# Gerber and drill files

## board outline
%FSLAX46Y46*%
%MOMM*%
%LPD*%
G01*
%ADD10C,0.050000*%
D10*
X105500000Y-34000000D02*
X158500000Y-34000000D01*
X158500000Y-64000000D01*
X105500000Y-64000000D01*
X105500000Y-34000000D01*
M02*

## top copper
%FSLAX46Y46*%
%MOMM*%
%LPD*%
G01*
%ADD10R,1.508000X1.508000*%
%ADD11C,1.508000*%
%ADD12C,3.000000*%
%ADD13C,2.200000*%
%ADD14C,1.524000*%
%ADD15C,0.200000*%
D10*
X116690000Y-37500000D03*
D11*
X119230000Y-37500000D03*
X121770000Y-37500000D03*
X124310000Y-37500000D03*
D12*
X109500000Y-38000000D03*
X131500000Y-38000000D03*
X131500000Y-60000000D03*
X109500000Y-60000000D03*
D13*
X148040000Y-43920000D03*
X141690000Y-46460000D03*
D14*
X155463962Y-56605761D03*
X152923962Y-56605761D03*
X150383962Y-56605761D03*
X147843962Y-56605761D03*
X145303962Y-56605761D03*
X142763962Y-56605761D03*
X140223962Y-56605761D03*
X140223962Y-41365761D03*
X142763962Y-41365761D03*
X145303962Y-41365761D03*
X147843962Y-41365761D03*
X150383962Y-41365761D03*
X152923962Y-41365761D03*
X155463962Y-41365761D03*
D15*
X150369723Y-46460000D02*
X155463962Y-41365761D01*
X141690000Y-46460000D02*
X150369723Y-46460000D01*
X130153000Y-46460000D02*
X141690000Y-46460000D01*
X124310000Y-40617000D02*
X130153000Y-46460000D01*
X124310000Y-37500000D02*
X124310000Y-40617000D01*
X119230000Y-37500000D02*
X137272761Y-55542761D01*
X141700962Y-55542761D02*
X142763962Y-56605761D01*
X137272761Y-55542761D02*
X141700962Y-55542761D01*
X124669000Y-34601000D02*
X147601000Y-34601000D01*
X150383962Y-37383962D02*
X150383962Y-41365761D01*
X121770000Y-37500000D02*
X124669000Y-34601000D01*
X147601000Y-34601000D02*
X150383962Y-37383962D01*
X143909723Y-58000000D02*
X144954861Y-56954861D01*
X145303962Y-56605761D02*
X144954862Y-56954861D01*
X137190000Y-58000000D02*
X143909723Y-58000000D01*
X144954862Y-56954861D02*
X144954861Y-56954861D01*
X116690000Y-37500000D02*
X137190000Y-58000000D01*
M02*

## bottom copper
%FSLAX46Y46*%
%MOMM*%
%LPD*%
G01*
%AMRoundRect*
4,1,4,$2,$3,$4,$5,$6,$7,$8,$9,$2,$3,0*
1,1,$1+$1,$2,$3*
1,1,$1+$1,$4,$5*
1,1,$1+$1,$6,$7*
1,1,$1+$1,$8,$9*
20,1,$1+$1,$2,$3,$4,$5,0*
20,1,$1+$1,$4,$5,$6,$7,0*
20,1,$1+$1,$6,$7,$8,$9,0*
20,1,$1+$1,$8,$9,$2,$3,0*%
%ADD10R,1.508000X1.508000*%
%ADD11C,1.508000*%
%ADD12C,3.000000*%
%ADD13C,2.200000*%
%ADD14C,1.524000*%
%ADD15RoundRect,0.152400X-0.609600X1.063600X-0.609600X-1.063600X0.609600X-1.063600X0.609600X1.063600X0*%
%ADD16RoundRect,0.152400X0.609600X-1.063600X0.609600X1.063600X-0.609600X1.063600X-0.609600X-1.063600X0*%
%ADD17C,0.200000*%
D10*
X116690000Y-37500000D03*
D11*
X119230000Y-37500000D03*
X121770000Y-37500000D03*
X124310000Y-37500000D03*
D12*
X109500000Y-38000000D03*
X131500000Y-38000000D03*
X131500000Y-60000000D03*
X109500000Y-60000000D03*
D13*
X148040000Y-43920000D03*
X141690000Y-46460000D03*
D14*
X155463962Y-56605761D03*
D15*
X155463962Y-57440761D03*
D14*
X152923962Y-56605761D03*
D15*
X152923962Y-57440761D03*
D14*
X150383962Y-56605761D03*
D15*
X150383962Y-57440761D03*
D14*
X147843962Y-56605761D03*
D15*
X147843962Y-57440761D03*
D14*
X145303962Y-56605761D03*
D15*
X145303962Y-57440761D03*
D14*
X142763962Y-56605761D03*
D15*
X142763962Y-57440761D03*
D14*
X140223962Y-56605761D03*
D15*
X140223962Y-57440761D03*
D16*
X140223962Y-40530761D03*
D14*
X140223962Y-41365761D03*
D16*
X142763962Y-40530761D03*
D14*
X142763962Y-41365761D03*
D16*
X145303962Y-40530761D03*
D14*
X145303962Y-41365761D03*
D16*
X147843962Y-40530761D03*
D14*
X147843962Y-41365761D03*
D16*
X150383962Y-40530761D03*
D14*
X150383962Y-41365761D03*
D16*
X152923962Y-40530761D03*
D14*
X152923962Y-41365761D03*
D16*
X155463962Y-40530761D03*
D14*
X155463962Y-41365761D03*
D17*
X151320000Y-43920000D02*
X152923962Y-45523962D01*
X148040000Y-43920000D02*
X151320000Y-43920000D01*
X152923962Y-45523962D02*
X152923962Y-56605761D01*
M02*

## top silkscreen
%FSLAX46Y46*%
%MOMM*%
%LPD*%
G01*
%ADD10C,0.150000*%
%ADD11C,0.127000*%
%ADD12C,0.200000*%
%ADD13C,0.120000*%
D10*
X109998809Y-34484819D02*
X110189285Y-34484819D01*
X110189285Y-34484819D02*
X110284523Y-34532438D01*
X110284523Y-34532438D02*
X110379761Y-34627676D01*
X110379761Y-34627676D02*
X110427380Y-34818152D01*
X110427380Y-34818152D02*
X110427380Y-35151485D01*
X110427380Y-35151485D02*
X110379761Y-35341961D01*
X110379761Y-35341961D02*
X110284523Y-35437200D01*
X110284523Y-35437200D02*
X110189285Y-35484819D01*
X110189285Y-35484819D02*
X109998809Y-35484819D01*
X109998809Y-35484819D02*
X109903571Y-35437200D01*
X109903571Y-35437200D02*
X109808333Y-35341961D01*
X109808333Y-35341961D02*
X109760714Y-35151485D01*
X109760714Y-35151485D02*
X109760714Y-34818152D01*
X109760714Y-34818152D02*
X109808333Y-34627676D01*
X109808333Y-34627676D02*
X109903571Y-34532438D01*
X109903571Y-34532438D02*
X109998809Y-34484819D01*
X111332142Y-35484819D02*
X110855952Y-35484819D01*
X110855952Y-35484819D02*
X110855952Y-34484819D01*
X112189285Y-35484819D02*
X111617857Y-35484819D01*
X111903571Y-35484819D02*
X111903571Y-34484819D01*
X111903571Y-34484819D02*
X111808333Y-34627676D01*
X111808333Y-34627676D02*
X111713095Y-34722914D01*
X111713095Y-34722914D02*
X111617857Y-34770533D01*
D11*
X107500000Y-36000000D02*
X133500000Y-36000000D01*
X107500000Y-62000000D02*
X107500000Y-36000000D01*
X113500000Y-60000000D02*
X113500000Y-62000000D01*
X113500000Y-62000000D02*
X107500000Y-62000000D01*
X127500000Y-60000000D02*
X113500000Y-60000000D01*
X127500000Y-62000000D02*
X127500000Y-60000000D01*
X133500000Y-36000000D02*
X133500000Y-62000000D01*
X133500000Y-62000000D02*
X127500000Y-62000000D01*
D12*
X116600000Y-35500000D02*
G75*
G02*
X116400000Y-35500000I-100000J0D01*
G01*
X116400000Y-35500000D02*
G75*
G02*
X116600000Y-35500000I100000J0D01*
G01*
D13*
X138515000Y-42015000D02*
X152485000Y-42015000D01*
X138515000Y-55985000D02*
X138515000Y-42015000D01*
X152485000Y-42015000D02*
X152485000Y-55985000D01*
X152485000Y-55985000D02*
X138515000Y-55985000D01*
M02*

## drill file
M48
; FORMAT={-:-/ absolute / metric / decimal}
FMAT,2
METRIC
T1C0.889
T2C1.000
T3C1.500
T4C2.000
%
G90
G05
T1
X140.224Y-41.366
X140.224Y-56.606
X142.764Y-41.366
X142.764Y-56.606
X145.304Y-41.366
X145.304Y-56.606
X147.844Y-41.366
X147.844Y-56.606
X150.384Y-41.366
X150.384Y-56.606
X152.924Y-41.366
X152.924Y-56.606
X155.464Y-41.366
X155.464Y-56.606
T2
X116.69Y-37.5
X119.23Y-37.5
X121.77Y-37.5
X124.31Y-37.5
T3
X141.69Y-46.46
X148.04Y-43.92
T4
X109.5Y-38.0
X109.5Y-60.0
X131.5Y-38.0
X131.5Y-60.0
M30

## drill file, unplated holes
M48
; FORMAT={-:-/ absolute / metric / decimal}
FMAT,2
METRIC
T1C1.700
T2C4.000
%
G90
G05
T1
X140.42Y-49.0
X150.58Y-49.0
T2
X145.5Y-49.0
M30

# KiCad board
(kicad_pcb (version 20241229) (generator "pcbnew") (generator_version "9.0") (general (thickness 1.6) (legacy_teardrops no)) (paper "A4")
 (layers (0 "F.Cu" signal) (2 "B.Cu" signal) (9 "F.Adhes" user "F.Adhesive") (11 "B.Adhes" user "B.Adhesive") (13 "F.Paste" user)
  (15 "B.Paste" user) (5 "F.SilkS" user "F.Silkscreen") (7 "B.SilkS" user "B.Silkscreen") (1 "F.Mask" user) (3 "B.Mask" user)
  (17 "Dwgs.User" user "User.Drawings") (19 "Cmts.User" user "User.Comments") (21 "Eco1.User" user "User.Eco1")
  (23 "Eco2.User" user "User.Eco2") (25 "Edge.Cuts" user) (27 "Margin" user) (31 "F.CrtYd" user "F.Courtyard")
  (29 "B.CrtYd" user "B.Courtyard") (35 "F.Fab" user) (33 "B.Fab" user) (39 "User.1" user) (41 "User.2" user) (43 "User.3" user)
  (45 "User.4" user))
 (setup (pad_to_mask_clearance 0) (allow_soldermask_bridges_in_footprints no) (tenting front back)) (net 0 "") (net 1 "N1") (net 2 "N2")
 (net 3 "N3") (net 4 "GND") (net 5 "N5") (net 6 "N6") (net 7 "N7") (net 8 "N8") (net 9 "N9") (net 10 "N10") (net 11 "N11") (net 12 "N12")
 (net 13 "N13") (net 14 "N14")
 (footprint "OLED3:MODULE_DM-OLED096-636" (layer "F.Cu") (at 120.5 49)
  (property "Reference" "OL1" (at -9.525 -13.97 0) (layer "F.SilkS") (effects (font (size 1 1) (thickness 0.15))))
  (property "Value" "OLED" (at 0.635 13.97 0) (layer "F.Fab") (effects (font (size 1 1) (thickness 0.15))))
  (fp_line (start -13 -13) (end 13 -13) (stroke (width 0.127) (type solid)) (layer "F.SilkS"))
  (fp_line (start -13 13) (end -13 -13) (stroke (width 0.127) (type solid)) (layer "F.SilkS"))
  (fp_line (start -7 11) (end -7 13) (stroke (width 0.127) (type solid)) (layer "F.SilkS"))
  (fp_line (start -7 13) (end -13 13) (stroke (width 0.127) (type solid)) (layer "F.SilkS"))
  (fp_line (start 7 11) (end -7 11) (stroke (width 0.127) (type solid)) (layer "F.SilkS"))
  (fp_line (start 7 13) (end 7 11) (stroke (width 0.127) (type solid)) (layer "F.SilkS"))
  (fp_line (start 13 -13) (end 13 13) (stroke (width 0.127) (type solid)) (layer "F.SilkS"))
  (fp_line (start 13 13) (end 7 13) (stroke (width 0.127) (type solid)) (layer "F.SilkS"))
  (fp_circle (center -4 -13.5) (end -3.9 -13.5) (stroke (width 0.2) (type solid)) (fill no) (layer "F.SilkS"))
  (pad "1" thru_hole rect (at -3.81 -11.5) (size 1.508 1.508) (drill 1) (layers "*.Cu" "*.Mask") (remove_unused_layers no) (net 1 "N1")
   (solder_mask_margin 0.102))
  (pad "2" thru_hole circle (at -1.27 -11.5) (size 1.508 1.508) (drill 1) (layers "*.Cu" "*.Mask") (remove_unused_layers no) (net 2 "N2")
   (solder_mask_margin 0.102))
  (pad "3" thru_hole circle (at 1.27 -11.5) (size 1.508 1.508) (drill 1) (layers "*.Cu" "*.Mask") (remove_unused_layers no) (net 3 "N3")
   (solder_mask_margin 0.102))
  (pad "4" thru_hole circle (at 3.81 -11.5) (size 1.508 1.508) (drill 1) (layers "*.Cu" "*.Mask") (remove_unused_layers no) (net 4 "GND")
   (solder_mask_margin 0.102))
  (pad "S1" thru_hole circle (at -11 -11) (size 3 3) (drill 2) (layers "*.Cu" "*.Mask") (remove_unused_layers no) (solder_mask_margin 0.102))
  (pad "S2" thru_hole circle (at 11 -11) (size 3 3) (drill 2) (layers "*.Cu" "*.Mask") (remove_unused_layers no) (solder_mask_margin 0.102))
  (pad "S3" thru_hole circle (at 11 11) (size 3 3) (drill 2) (layers "*.Cu" "*.Mask") (remove_unused_layers no) (solder_mask_margin 0.102))
  (pad "S4" thru_hole circle (at -11 11) (size 3 3) (drill 2) (layers "*.Cu" "*.Mask") (remove_unused_layers no) (solder_mask_margin 0.102)))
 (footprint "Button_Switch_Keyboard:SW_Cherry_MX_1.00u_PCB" (layer "F.Cu") (at 148.04 43.92)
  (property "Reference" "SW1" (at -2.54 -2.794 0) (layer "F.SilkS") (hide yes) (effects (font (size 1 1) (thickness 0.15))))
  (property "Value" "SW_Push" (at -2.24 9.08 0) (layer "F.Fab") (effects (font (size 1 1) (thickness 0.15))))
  (fp_line (start -9.525 -1.905) (end 4.445 -1.905) (stroke (width 0.12) (type solid)) (layer "F.SilkS"))
  (fp_line (start -9.525 12.065) (end -9.525 -1.905) (stroke (width 0.12) (type solid)) (layer "F.SilkS"))
  (fp_line (start 4.445 -1.905) (end 4.445 12.065) (stroke (width 0.12) (type solid)) (layer "F.SilkS"))
  (fp_line (start 4.445 12.065) (end -9.525 12.065) (stroke (width 0.12) (type solid)) (layer "F.SilkS"))
  (pad "" np_thru_hole circle (at -7.62 5.08) (size 1.7 1.7) (drill 1.7) (layers "*.Cu" "*.Mask"))
  (pad "" np_thru_hole circle (at -2.54 5.08) (size 4 4) (drill 4) (layers "*.Cu" "*.Mask"))
  (pad "" np_thru_hole circle (at 2.54 5.08) (size 1.7 1.7) (drill 1.7) (layers "*.Cu" "*.Mask"))
  (pad "1" thru_hole circle (at 0 0) (size 2.2 2.2) (drill 1.5) (layers "*.Cu" "*.Mask") (remove_unused_layers no) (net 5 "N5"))
  (pad "2" thru_hole circle (at -6.35 2.54) (size 2.2 2.2) (drill 1.5) (layers "*.Cu" "*.Mask") (remove_unused_layers no) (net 4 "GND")))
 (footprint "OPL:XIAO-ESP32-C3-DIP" (layer "B.Cu") (at 147.843962 48.985761)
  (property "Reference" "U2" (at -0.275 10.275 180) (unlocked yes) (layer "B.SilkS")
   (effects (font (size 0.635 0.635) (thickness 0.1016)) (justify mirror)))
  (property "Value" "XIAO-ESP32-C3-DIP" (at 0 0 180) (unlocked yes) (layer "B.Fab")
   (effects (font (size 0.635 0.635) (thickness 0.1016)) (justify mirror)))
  (pad "1" thru_hole circle (at 7.62 7.62 270) (size 1.524 1.524) (drill 0.889) (layers "*.Cu" "*.Mask") (remove_unused_layers no)
   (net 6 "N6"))
  (pad "1" smd roundrect (at 7.62 8.455 270) (size 2.432 1.524) (layers "B.Cu" "B.Mask") (roundrect_rratio 0.1) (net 6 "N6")
   (thermal_bridge_angle 45))
  (pad "2" thru_hole circle (at 5.08 7.62 270) (size 1.524 1.524) (drill 0.889) (layers "*.Cu" "*.Mask") (remove_unused_layers no)
   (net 5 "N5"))
  (pad "2" smd roundrect (at 5.08 8.455 270) (size 2.432 1.524) (layers "B.Cu" "B.Mask") (roundrect_rratio 0.1) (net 5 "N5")
   (thermal_bridge_angle 45))
  (pad "3" thru_hole circle (at 2.54 7.62 270) (size 1.524 1.524) (drill 0.889) (layers "*.Cu" "*.Mask") (remove_unused_layers no)
   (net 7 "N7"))
  (pad "3" smd roundrect (at 2.54 8.455 270) (size 2.432 1.524) (layers "B.Cu" "B.Mask") (roundrect_rratio 0.1) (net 7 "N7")
   (thermal_bridge_angle 45))
  (pad "4" thru_hole circle (at 0 7.62 270) (size 1.524 1.524) (drill 0.889) (layers "*.Cu" "*.Mask") (remove_unused_layers no) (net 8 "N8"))
  (pad "4" smd roundrect (at 0 8.455 270) (size 2.432 1.524) (layers "B.Cu" "B.Mask") (roundrect_rratio 0.1) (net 8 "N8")
   (thermal_bridge_angle 45))
  (pad "5" thru_hole circle (at -2.54 7.62 270) (size 1.524 1.524) (drill 0.889) (layers "*.Cu" "*.Mask") (remove_unused_layers no)
   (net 1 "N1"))
  (pad "5" smd roundrect (at -2.54 8.455 270) (size 2.432 1.524) (layers "B.Cu" "B.Mask") (roundrect_rratio 0.1) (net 1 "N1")
   (thermal_bridge_angle 45))
  (pad "6" thru_hole circle (at -5.08 7.62 270) (size 1.524 1.524) (drill 0.889) (layers "*.Cu" "*.Mask") (remove_unused_layers no)
   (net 2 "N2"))
  (pad "6" smd roundrect (at -5.08 8.455 270) (size 2.432 1.524) (layers "B.Cu" "B.Mask") (roundrect_rratio 0.1) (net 2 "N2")
   (thermal_bridge_angle 45))
  (pad "7" thru_hole circle (at -7.62 7.62 270) (size 1.524 1.524) (drill 0.889) (layers "*.Cu" "*.Mask") (remove_unused_layers no)
   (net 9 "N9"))
  (pad "7" smd roundrect (at -7.62 8.455 270) (size 2.432 1.524) (layers "B.Cu" "B.Mask") (roundrect_rratio 0.1) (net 9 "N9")
   (thermal_bridge_angle 45))
  (pad "8" smd roundrect (at -7.62 -8.455 90) (size 2.432 1.524) (layers "B.Cu" "B.Mask") (roundrect_rratio 0.1) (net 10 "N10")
   (thermal_bridge_angle 45))
  (pad "8" thru_hole circle (at -7.62 -7.62 90) (size 1.524 1.524) (drill 0.889) (layers "*.Cu" "*.Mask") (remove_unused_layers no)
   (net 10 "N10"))
  (pad "9" smd roundrect (at -5.08 -8.455 90) (size 2.432 1.524) (layers "B.Cu" "B.Mask") (roundrect_rratio 0.1) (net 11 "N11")
   (thermal_bridge_angle 45))
  (pad "9" thru_hole circle (at -5.08 -7.62 90) (size 1.524 1.524) (drill 0.889) (layers "*.Cu" "*.Mask") (remove_unused_layers no)
   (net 11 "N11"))
  (pad "10" smd roundrect (at -2.54 -8.455 90) (size 2.432 1.524) (layers "B.Cu" "B.Mask") (roundrect_rratio 0.1) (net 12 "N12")
   (thermal_bridge_angle 45))
  (pad "10" thru_hole circle (at -2.54 -7.62 90) (size 1.524 1.524) (drill 0.889) (layers "*.Cu" "*.Mask") (remove_unused_layers no)
   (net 12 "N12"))
  (pad "11" smd roundrect (at 0 -8.455 90) (size 2.432 1.524) (layers "B.Cu" "B.Mask") (roundrect_rratio 0.1) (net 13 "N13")
   (thermal_bridge_angle 45))
  (pad "11" thru_hole circle (at 0 -7.62 90) (size 1.524 1.524) (drill 0.889) (layers "*.Cu" "*.Mask") (remove_unused_layers no)
   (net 13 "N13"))
  (pad "12" smd roundrect (at 2.54 -8.455 90) (size 2.432 1.524) (layers "B.Cu" "B.Mask") (roundrect_rratio 0.1) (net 3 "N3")
   (thermal_bridge_angle 45))
  (pad "12" thru_hole circle (at 2.54 -7.62 90) (size 1.524 1.524) (drill 0.889) (layers "*.Cu" "*.Mask") (remove_unused_layers no)
   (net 3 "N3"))
  (pad "13" smd roundrect (at 5.08 -8.455 90) (size 2.432 1.524) (layers "B.Cu" "B.Mask") (roundrect_rratio 0.1) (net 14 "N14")
   (thermal_bridge_angle 45))
  (pad "13" thru_hole circle (at 5.08 -7.62 90) (size 1.524 1.524) (drill 0.889) (layers "*.Cu" "*.Mask") (remove_unused_layers no)
   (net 14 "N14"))
  (pad "14" smd roundrect (at 7.62 -8.455 90) (size 2.432 1.524) (layers "B.Cu" "B.Mask") (roundrect_rratio 0.1) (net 4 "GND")
   (thermal_bridge_angle 45))
  (pad "14" thru_hole circle (at 7.62 -7.62 90) (size 1.524 1.524) (drill 0.889) (layers "*.Cu" "*.Mask") (remove_unused_layers no)
   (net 4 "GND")))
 (gr_rect (start 105.5 34) (end 158.5 64) (stroke (width 0.05) (type default)) (fill no) (layer "Edge.Cuts"))
 (segment (start 119.23 37.5) (end 137.272761 55.542761) (width 0.2) (layer "F.Cu") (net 2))
 (segment (start 141.700962 55.542761) (end 142.763962 56.605761) (width 0.2) (layer "F.Cu") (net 2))
 (segment (start 137.272761 55.542761) (end 141.700962 55.542761) (width 0.2) (layer "F.Cu") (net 2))
 (segment (start 124.669 34.601) (end 147.601 34.601) (width 0.2) (layer "F.Cu") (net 3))
 (segment (start 150.383962 37.383962) (end 150.383962 41.365761) (width 0.2) (layer "F.Cu") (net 3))
 (segment (start 121.77 37.5) (end 124.669 34.601) (width 0.2) (layer "F.Cu") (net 3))
 (segment (start 147.601 34.601) (end 150.383962 37.383962) (width 0.2) (layer "F.Cu") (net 3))
 (segment (start 143.909723 58) (end 144.954861 56.954861) (width 0.2) (layer "F.Cu") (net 1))
 (segment (start 145.303962 56.605761) (end 144.954862 56.954861) (width 0.2) (layer "F.Cu") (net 1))
 (segment (start 137.19 58) (end 143.909723 58) (width 0.2) (layer "F.Cu") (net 1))
 (segment (start 144.954862 56.954861) (end 144.954861 56.954861) (width 0.2) (layer "F.Cu") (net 1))
 (segment (start 116.69 37.5) (end 137.19 58) (width 0.2) (layer "F.Cu") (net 1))
 (segment (start 151.32 43.92) (end 152.923962 45.523962) (width 0.2) (layer "B.Cu") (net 5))
 (segment (start 148.04 43.92) (end 151.32 43.92) (width 0.2) (layer "B.Cu") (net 5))
 (segment (start 152.923962 45.523962) (end 152.923962 56.605761) (width 0.2) (layer "B.Cu") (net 5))
 (segment (start 141.69 46.46) (end 150.369723 46.46) (width 0.2) (layer "F.Cu") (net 4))
 (segment (start 130.153 46.46) (end 141.69 46.46) (width 0.2) (layer "F.Cu") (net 4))
 (segment (start 124.31 37.5) (end 124.31 40.617) (width 0.2) (layer "F.Cu") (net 4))
 (segment (start 150.369723 46.46) (end 155.463962 41.365761) (width 0.2) (layer "F.Cu") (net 4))
 (segment (start 124.31 40.617) (end 130.153 46.46) (width 0.2) (layer "F.Cu") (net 4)))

